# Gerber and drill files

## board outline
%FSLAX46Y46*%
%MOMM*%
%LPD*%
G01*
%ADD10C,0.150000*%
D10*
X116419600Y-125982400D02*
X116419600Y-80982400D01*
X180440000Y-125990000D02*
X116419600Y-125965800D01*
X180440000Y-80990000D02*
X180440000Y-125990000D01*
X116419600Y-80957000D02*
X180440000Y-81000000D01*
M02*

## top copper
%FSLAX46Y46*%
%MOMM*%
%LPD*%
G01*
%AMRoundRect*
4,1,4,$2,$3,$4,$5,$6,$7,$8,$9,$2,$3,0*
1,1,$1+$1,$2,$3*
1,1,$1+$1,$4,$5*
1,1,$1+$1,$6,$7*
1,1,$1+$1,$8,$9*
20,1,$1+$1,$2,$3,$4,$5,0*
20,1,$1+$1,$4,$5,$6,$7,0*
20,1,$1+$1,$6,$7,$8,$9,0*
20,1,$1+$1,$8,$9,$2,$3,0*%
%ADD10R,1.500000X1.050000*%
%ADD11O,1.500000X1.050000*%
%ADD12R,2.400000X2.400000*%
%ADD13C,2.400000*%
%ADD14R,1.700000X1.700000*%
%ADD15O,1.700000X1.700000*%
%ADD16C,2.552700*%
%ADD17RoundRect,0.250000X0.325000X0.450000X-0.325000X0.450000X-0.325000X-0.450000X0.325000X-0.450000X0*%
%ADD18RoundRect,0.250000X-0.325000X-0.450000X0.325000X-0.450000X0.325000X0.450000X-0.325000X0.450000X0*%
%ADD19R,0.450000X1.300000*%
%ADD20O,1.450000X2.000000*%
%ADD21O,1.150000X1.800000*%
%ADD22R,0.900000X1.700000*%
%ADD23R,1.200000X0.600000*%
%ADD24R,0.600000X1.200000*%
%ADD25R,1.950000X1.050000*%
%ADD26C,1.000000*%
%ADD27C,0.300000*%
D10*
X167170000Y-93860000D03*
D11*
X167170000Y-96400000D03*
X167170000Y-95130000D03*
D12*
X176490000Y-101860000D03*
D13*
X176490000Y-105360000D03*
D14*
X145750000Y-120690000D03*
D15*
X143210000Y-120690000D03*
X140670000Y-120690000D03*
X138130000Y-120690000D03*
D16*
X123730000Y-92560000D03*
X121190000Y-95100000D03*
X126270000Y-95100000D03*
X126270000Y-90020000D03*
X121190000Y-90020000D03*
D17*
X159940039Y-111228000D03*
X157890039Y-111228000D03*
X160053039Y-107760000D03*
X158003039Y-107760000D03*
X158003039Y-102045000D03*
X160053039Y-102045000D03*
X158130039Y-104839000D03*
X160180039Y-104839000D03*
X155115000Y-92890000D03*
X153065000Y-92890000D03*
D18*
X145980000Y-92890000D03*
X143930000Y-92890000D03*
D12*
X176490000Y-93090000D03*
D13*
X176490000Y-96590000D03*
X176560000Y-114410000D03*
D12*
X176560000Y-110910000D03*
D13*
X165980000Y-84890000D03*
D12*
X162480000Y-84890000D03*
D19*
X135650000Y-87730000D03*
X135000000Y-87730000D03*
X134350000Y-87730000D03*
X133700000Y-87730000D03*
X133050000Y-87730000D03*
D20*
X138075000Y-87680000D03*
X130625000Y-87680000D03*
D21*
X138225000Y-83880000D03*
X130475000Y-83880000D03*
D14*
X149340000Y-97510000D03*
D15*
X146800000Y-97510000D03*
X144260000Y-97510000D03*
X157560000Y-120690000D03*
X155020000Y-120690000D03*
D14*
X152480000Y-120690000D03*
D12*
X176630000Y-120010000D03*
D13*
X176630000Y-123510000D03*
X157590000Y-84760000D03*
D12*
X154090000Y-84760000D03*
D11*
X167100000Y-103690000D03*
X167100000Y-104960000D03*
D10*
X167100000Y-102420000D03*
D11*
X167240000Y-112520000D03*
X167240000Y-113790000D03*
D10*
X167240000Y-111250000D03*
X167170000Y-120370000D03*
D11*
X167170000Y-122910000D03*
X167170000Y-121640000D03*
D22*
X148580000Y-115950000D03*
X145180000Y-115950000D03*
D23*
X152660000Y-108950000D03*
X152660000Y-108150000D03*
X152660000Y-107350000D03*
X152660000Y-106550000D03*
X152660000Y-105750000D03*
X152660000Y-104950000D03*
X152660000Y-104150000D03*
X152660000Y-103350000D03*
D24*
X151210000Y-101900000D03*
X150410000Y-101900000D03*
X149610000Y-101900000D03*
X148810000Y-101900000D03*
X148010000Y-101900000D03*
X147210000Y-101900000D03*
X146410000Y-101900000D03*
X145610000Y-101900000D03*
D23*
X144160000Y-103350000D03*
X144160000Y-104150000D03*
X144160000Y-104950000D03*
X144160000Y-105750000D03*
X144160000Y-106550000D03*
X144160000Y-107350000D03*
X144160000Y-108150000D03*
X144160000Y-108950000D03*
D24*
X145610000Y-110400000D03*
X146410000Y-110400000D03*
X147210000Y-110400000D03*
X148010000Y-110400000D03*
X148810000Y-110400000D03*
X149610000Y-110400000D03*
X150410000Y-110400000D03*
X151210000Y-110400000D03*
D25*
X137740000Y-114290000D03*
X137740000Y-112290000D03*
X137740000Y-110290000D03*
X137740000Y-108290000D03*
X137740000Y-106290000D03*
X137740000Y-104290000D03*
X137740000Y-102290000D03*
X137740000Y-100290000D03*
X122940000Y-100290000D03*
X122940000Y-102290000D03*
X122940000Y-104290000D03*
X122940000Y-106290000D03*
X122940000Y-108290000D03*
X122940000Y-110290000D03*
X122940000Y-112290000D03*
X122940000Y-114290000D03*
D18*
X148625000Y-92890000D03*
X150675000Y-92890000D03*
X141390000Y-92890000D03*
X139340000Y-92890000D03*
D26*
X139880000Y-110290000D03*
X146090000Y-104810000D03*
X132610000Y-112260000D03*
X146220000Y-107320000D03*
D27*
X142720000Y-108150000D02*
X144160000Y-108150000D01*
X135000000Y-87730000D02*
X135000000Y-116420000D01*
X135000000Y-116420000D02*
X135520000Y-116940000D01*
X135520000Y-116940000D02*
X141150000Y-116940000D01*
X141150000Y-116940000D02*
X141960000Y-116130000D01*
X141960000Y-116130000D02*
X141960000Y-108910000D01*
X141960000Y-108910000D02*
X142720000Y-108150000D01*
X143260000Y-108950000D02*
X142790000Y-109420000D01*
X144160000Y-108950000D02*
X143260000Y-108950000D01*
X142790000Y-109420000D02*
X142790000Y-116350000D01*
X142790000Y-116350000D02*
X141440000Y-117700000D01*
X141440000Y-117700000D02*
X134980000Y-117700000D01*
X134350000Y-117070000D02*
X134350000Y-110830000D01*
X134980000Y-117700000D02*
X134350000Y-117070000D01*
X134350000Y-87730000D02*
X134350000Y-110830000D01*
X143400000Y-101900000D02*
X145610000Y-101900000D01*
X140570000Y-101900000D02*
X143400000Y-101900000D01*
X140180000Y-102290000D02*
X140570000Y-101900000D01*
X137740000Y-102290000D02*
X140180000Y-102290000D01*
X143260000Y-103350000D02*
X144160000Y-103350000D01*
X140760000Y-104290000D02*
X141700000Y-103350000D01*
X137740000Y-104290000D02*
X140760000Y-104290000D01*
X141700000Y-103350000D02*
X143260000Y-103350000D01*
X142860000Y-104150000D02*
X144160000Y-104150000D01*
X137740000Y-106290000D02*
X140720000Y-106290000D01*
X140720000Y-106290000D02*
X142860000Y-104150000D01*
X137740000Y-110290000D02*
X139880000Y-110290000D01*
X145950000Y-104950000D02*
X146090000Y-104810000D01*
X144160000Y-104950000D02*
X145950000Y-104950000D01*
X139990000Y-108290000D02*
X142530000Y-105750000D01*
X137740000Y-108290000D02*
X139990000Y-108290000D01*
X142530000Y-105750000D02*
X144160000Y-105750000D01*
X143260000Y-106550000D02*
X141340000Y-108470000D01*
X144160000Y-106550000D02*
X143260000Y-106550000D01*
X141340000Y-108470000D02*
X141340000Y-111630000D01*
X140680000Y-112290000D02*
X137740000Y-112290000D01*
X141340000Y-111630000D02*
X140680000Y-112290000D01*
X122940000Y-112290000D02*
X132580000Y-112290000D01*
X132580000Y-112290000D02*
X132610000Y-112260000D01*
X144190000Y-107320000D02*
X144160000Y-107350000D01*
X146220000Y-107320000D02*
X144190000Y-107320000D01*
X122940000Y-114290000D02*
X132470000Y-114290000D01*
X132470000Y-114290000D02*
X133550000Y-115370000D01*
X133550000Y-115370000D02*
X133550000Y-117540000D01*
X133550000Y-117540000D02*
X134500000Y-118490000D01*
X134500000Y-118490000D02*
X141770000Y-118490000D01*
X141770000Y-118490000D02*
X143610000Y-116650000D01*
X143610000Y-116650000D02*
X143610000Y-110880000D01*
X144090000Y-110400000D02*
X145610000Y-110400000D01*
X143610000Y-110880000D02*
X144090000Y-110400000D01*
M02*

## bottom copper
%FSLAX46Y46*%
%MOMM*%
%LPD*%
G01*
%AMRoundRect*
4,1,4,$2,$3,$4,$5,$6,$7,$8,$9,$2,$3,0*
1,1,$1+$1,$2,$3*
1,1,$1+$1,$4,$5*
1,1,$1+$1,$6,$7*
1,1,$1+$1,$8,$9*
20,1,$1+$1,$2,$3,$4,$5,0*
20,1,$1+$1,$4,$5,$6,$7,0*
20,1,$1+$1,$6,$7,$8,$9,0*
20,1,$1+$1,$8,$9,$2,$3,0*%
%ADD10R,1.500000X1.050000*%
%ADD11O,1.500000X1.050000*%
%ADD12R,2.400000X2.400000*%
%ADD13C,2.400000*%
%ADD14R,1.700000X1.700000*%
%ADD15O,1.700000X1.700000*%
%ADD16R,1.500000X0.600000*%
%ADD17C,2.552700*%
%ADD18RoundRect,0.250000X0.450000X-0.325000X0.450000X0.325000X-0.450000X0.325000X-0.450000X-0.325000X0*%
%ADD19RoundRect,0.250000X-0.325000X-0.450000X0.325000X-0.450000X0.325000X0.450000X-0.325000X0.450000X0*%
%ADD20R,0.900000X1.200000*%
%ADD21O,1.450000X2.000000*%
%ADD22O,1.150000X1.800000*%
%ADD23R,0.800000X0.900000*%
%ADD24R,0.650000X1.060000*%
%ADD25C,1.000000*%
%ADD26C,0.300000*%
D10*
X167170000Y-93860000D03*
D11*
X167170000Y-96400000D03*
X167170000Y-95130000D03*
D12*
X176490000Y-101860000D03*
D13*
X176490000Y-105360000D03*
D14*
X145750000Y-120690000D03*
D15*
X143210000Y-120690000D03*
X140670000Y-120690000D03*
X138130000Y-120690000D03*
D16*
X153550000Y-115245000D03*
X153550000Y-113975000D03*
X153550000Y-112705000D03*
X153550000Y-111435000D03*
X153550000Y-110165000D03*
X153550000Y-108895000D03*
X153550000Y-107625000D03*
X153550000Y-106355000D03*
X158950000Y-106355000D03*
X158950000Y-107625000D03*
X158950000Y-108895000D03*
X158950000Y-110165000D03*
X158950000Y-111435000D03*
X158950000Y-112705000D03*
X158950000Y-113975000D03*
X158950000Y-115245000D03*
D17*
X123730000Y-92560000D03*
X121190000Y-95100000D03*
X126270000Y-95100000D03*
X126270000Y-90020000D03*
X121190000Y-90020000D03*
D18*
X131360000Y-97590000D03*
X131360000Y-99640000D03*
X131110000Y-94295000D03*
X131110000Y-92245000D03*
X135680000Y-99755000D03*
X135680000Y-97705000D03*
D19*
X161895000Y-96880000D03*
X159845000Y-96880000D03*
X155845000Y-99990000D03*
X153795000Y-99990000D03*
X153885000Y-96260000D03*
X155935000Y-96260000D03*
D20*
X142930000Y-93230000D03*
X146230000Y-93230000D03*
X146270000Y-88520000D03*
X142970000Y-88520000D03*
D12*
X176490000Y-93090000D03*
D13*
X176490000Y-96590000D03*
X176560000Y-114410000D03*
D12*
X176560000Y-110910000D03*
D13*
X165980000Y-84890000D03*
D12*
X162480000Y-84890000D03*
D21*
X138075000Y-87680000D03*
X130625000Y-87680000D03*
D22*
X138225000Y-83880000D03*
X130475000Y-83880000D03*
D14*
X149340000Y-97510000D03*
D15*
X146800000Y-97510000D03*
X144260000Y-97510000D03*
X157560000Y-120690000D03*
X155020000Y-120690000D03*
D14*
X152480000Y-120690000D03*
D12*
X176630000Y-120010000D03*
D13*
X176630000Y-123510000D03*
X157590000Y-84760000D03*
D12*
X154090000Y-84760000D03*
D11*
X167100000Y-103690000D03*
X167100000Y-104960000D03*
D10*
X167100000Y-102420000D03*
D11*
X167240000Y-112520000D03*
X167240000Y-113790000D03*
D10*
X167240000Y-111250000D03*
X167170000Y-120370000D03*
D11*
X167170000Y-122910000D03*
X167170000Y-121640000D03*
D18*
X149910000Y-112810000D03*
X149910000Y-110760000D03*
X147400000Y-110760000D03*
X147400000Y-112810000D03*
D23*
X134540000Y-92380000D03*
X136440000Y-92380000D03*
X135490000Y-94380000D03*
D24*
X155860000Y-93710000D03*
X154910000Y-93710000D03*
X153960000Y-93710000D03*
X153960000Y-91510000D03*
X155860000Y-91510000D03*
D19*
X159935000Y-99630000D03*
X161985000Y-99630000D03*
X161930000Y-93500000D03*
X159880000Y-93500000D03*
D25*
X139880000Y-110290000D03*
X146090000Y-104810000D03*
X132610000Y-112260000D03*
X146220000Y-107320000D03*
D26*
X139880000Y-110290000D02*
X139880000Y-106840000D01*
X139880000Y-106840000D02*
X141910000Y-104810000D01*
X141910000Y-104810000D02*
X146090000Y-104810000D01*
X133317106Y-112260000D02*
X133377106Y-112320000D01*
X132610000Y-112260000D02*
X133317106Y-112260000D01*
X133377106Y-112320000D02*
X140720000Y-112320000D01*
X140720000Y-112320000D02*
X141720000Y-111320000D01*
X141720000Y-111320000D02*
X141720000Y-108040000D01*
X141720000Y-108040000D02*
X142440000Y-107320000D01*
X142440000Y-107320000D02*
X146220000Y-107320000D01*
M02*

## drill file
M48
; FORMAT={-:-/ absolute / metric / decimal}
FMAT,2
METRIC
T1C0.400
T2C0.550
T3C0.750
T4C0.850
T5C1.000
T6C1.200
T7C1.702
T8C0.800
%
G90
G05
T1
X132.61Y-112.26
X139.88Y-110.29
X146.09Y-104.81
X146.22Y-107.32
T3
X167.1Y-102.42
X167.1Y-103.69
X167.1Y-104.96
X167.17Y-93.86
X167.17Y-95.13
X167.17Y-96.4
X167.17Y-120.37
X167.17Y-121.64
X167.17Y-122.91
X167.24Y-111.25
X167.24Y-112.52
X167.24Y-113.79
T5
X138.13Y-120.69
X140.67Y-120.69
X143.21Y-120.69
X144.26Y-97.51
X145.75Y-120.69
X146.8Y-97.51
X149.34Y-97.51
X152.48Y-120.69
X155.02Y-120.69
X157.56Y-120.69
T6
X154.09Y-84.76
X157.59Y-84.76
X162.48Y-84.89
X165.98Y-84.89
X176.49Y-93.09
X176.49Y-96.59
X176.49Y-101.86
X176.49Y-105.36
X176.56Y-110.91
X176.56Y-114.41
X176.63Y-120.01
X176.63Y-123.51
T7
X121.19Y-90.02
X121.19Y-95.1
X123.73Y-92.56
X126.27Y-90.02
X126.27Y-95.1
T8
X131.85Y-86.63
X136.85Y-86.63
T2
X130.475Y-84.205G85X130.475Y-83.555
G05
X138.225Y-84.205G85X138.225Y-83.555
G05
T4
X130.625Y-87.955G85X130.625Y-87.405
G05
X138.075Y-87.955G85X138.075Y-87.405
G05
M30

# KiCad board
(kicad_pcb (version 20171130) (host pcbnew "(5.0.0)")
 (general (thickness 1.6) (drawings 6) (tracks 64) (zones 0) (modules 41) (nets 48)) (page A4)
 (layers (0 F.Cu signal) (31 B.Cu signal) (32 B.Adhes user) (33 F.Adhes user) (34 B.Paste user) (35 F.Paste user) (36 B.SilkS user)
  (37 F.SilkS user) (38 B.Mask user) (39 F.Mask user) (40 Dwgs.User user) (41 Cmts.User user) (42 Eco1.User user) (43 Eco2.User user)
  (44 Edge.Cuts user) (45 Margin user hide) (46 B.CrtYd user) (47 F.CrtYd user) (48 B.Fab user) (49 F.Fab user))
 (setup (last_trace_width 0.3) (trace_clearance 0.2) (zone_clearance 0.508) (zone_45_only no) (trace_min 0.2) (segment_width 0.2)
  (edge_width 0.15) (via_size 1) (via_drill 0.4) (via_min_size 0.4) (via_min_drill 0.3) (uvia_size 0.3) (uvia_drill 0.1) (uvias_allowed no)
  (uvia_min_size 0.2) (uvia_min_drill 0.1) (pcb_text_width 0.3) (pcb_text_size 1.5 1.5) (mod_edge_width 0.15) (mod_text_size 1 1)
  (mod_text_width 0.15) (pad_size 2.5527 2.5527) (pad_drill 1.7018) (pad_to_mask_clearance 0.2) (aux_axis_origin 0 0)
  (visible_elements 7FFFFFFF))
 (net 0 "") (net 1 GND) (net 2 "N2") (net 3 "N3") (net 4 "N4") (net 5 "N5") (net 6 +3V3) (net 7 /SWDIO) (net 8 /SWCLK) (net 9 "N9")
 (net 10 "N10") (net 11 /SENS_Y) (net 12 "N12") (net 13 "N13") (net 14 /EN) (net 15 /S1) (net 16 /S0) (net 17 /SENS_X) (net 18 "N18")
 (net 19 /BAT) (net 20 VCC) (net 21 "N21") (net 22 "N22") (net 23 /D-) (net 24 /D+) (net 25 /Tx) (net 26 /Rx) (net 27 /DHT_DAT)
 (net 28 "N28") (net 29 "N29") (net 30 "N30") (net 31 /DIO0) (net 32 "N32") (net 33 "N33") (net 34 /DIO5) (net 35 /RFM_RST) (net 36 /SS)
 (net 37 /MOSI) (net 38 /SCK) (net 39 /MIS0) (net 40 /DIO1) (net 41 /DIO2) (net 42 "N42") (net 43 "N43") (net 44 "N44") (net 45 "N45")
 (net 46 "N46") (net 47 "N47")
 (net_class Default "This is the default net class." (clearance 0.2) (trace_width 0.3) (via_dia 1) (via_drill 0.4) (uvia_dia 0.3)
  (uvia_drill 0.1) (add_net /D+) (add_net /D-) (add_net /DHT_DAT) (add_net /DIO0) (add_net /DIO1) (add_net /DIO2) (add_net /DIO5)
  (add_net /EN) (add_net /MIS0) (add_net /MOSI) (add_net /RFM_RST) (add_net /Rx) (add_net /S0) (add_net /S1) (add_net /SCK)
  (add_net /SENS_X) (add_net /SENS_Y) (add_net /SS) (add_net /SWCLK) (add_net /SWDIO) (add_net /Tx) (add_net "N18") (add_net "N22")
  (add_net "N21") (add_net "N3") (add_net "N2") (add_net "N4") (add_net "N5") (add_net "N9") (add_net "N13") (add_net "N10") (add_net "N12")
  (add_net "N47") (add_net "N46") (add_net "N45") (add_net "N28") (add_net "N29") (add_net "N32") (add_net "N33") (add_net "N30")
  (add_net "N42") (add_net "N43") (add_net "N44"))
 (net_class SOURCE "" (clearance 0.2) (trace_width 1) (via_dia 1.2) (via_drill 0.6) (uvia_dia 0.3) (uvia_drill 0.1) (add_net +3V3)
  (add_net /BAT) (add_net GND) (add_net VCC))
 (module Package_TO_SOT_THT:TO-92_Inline (layer F.Cu) (at 167.17 93.86 270)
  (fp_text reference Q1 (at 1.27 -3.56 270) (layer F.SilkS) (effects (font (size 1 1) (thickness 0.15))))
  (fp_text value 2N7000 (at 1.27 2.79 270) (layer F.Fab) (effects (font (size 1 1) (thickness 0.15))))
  (pad 1 thru_hole rect (at 0 0 270) (size 1.05 1.5) (drill 0.75) (layers *.Cu *.Mask) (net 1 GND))
  (pad 3 thru_hole oval (at 2.54 0 270) (size 1.05 1.5) (drill 0.75) (layers *.Cu *.Mask) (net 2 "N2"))
  (pad 2 thru_hole oval (at 1.27 0 270) (size 1.05 1.5) (drill 0.75) (layers *.Cu *.Mask) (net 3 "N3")))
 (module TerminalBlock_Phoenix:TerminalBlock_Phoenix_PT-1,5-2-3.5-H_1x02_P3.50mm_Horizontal (layer F.Cu) (at 176.49 101.86 270)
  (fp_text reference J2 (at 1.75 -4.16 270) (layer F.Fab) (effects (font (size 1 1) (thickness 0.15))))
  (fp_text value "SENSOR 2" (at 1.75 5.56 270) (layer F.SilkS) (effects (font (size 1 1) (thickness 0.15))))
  (pad 1 thru_hole rect (at 0 0 270) (size 2.4 2.4) (drill 1.2) (layers *.Cu *.Mask) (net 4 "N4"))
  (pad 2 thru_hole circle (at 3.5 0 270) (size 2.4 2.4) (drill 1.2) (layers *.Cu *.Mask) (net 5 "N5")))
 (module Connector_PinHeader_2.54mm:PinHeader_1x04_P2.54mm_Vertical (layer F.Cu) (at 145.75 120.69 270)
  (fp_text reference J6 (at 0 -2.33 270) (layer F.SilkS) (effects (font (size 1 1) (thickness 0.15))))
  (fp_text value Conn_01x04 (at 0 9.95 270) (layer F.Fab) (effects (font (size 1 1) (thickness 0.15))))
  (pad 1 thru_hole rect (at 0 0 270) (size 1.7 1.7) (drill 1) (layers *.Cu *.Mask) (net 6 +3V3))
  (pad 2 thru_hole oval (at 0 2.54 270) (size 1.7 1.7) (drill 1) (layers *.Cu *.Mask) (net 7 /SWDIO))
  (pad 3 thru_hole oval (at 0 5.08 270) (size 1.7 1.7) (drill 1) (layers *.Cu *.Mask) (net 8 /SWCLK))
  (pad 4 thru_hole oval (at 0 7.62 270) (size 1.7 1.7) (drill 1) (layers *.Cu *.Mask) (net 1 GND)))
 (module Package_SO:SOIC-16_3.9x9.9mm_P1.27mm (layer B.Cu) (at 156.25 110.8)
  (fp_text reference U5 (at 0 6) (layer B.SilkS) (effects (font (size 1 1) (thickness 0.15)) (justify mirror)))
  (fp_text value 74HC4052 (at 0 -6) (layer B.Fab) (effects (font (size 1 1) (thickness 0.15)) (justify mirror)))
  (pad 1 smd rect (at -2.7 4.445) (size 1.5 0.6) (layers B.Cu B.Paste B.Mask) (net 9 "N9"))
  (pad 2 smd rect (at -2.7 3.175) (size 1.5 0.6) (layers B.Cu B.Paste B.Mask) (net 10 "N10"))
  (pad 3 smd rect (at -2.7 1.905) (size 1.5 0.6) (layers B.Cu B.Paste B.Mask) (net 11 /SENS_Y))
  (pad 4 smd rect (at -2.7 0.635) (size 1.5 0.6) (layers B.Cu B.Paste B.Mask) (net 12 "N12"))
  (pad 5 smd rect (at -2.7 -0.635) (size 1.5 0.6) (layers B.Cu B.Paste B.Mask) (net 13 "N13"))
  (pad 6 smd rect (at -2.7 -1.905) (size 1.5 0.6) (layers B.Cu B.Paste B.Mask) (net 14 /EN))
  (pad 7 smd rect (at -2.7 -3.175) (size 1.5 0.6) (layers B.Cu B.Paste B.Mask) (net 1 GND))
  (pad 8 smd rect (at -2.7 -4.445) (size 1.5 0.6) (layers B.Cu B.Paste B.Mask) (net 1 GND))
  (pad 9 smd rect (at 2.7 -4.445) (size 1.5 0.6) (layers B.Cu B.Paste B.Mask) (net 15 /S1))
  (pad 10 smd rect (at 2.7 -3.175) (size 1.5 0.6) (layers B.Cu B.Paste B.Mask) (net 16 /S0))
  (pad 11 smd rect (at 2.7 -1.905) (size 1.5 0.6) (layers B.Cu B.Paste B.Mask) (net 5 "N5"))
  (pad 12 smd rect (at 2.7 -0.635) (size 1.5 0.6) (layers B.Cu B.Paste B.Mask) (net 3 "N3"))
  (pad 13 smd rect (at 2.7 0.635) (size 1.5 0.6) (layers B.Cu B.Paste B.Mask) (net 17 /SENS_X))
  (pad 14 smd rect (at 2.7 1.905) (size 1.5 0.6) (layers B.Cu B.Paste B.Mask) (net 2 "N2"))
  (pad 15 smd rect (at 2.7 3.175) (size 1.5 0.6) (layers B.Cu B.Paste B.Mask) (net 4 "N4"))
  (pad 16 smd rect (at 2.7 4.445) (size 1.5 0.6) (layers B.Cu B.Paste B.Mask) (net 6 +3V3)))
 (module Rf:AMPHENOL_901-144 (layer F.Cu) (at 123.73 92.56 90) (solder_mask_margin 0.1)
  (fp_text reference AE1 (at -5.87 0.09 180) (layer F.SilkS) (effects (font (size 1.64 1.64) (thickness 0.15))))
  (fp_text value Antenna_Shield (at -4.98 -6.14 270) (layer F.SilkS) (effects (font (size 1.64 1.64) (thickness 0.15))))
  (pad 1 thru_hole circle (at 0 0 90) (size 2.5527 2.5527) (drill 1.7018) (layers *.Cu *.Mask F.SilkS) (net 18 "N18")
   (solder_mask_margin 0.2))
  (pad 2 thru_hole circle (at -2.54 -2.54 90) (size 2.5527 2.5527) (drill 1.7018) (layers *.Cu *.Mask F.SilkS) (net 1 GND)
   (solder_mask_margin 0.2))
  (pad E thru_hole circle (at -2.54 2.54 90) (size 2.5527 2.5527) (drill 1.7018) (layers *.Cu *.Mask F.SilkS) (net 1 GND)
   (solder_mask_margin 0.2))
  (pad 4 thru_hole circle (at 2.54 2.54 90) (size 2.5527 2.5527) (drill 1.7018) (layers *.Cu *.Mask F.SilkS) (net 1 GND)
   (solder_mask_margin 0.2))
  (pad 5 thru_hole circle (at 2.54 -2.54 90) (size 2.5527 2.5527) (drill 1.7018) (layers *.Cu *.Mask F.SilkS) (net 1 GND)
   (solder_mask_margin 0.2)))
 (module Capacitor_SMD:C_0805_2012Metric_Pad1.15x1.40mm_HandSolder (layer F.Cu) (at 158.915039 111.228 180)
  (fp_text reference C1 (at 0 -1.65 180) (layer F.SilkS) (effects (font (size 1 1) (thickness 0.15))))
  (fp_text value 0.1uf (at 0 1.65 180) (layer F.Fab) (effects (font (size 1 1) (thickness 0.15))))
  (pad 1 smd roundrect (at -1.025 0 180) (size 1.15 1.4) (layers F.Cu F.Paste F.Mask) (roundrect_rratio 0.217391) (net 6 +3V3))
  (pad 2 smd roundrect (at 1.025 0 180) (size 1.15 1.4) (layers F.Cu F.Paste F.Mask) (roundrect_rratio 0.217391) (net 1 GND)))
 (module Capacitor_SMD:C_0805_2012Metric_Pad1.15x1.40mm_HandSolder (layer B.Cu) (at 131.36 98.615 90)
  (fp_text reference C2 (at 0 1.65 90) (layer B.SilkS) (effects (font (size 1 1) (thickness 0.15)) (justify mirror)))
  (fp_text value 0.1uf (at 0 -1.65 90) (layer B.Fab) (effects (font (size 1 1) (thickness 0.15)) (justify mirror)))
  (pad 2 smd roundrect (at 1.025 0 90) (size 1.15 1.4) (layers B.Cu B.Paste B.Mask) (roundrect_rratio 0.217391) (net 1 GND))
  (pad 1 smd roundrect (at -1.025 0 90) (size 1.15 1.4) (layers B.Cu B.Paste B.Mask) (roundrect_rratio 0.217391) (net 6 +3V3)))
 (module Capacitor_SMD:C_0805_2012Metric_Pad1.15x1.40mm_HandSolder (layer F.Cu) (at 159.028039 107.76 180)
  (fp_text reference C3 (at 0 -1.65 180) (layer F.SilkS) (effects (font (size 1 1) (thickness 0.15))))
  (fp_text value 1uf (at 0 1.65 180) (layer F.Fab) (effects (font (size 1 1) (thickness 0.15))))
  (pad 1 smd roundrect (at -1.025 0 180) (size 1.15 1.4) (layers F.Cu F.Paste F.Mask) (roundrect_rratio 0.217391) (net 6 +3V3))
  (pad 2 smd roundrect (at 1.025 0 180) (size 1.15 1.4) (layers F.Cu F.Paste F.Mask) (roundrect_rratio 0.217391) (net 1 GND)))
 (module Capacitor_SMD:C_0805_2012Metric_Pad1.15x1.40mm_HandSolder (layer B.Cu) (at 131.11 93.27 90)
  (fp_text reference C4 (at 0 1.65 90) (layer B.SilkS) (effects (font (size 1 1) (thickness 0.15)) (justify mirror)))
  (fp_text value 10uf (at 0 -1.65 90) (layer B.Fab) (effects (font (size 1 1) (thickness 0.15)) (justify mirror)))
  (pad 1 smd roundrect (at -1.025 0 90) (size 1.15 1.4) (layers B.Cu B.Paste B.Mask) (roundrect_rratio 0.217391) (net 6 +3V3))
  (pad 2 smd roundrect (at 1.025 0 90) (size 1.15 1.4) (layers B.Cu B.Paste B.Mask) (roundrect_rratio 0.217391) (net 1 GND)))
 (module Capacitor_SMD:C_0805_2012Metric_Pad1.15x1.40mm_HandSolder (layer B.Cu) (at 135.68 98.73 90)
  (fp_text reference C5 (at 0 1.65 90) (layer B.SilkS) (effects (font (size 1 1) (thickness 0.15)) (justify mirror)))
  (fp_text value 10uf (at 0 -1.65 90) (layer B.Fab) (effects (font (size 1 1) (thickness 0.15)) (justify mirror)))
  (pad 1 smd roundrect (at -1.025 0 90) (size 1.15 1.4) (layers B.Cu B.Paste B.Mask) (roundrect_rratio 0.217391) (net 6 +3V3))
  (pad 2 smd roundrect (at 1.025 0 90) (size 1.15 1.4) (layers B.Cu B.Paste B.Mask) (roundrect_rratio 0.217391) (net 1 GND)))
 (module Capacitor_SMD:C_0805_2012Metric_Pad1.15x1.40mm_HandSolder (layer B.Cu) (at 160.87 96.88)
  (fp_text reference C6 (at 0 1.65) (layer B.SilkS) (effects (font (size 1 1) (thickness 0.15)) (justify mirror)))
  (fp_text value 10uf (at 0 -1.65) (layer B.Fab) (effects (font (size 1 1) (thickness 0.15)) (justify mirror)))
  (pad 2 smd roundrect (at 1.025 0) (size 1.15 1.4) (layers B.Cu B.Paste B.Mask) (roundrect_rratio 0.217391) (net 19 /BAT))
  (pad 1 smd roundrect (at -1.025 0) (size 1.15 1.4) (layers B.Cu B.Paste B.Mask) (roundrect_rratio 0.217391) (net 1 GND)))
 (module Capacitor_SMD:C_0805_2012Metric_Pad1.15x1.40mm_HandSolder (layer F.Cu) (at 159.028039 102.045 180)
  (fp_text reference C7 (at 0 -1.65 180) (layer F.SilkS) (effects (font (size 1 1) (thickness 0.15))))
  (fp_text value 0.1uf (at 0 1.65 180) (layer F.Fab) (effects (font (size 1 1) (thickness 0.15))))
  (pad 2 smd roundrect (at 1.025 0 180) (size 1.15 1.4) (layers F.Cu F.Paste F.Mask) (roundrect_rratio 0.217391) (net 1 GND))
  (pad 1 smd roundrect (at -1.025 0 180) (size 1.15 1.4) (layers F.Cu F.Paste F.Mask) (roundrect_rratio 0.217391) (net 6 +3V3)))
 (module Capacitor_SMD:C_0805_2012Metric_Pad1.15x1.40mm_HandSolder (layer F.Cu) (at 159.155039 104.839 180)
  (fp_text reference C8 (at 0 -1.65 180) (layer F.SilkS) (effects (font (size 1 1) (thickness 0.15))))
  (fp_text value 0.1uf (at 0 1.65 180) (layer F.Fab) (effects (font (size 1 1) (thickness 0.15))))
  (pad 2 smd roundrect (at 1.025 0 180) (size 1.15 1.4) (layers F.Cu F.Paste F.Mask) (roundrect_rratio 0.217391) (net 1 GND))
  (pad 1 smd roundrect (at -1.025 0 180) (size 1.15 1.4) (layers F.Cu F.Paste F.Mask) (roundrect_rratio 0.217391) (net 6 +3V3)))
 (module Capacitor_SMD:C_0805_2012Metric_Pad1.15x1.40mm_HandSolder (layer B.Cu) (at 154.82 99.99)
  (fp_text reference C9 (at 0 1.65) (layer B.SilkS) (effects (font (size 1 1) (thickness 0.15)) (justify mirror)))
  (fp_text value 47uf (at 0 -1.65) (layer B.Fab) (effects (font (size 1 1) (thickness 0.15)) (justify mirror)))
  (pad 2 smd roundrect (at 1.025 0) (size 1.15 1.4) (layers B.Cu B.Paste B.Mask) (roundrect_rratio 0.217391) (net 1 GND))
  (pad 1 smd roundrect (at -1.025 0) (size 1.15 1.4) (layers B.Cu B.Paste B.Mask) (roundrect_rratio 0.217391) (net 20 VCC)))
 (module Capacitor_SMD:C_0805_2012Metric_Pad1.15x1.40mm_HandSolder (layer B.Cu) (at 154.91 96.26)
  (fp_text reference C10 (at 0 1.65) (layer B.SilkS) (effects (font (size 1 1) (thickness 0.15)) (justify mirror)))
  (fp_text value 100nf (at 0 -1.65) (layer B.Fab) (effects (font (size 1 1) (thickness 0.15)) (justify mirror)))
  (pad 1 smd roundrect (at -1.025 0) (size 1.15 1.4) (layers B.Cu B.Paste B.Mask) (roundrect_rratio 0.217391) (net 20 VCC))
  (pad 2 smd roundrect (at 1.025 0) (size 1.15 1.4) (layers B.Cu B.Paste B.Mask) (roundrect_rratio 0.217391) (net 1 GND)))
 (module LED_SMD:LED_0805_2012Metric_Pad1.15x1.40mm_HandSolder (layer F.Cu) (at 154.09 92.89 180)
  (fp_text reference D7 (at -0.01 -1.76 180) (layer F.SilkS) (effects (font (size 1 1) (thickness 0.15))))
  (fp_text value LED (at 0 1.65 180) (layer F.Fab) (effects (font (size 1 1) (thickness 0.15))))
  (pad 1 smd roundrect (at -1.025 0 180) (size 1.15 1.4) (layers F.Cu F.Paste F.Mask) (roundrect_rratio 0.217391) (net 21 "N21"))
  (pad 2 smd roundrect (at 1.025 0 180) (size 1.15 1.4) (layers F.Cu F.Paste F.Mask) (roundrect_rratio 0.217391) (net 20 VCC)))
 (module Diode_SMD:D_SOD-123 (layer B.Cu) (at 144.58 93.23)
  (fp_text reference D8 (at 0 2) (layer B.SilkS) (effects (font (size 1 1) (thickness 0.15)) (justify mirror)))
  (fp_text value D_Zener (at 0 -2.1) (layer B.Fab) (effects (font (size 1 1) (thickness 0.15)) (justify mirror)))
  (pad 1 smd rect (at -1.65 0) (size 0.9 1.2) (layers B.Cu B.Paste B.Mask) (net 6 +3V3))
  (pad 2 smd rect (at 1.65 0) (size 0.9 1.2) (layers B.Cu B.Paste B.Mask) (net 20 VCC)))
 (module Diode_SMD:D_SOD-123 (layer B.Cu) (at 144.62 88.52)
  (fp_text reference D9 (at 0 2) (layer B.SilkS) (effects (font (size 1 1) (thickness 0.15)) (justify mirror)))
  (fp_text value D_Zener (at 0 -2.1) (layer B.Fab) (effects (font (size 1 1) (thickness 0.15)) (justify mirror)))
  (pad 2 smd rect (at 1.65 0) (size 0.9 1.2) (layers B.Cu B.Paste B.Mask) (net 19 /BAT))
  (pad 1 smd rect (at -1.65 0) (size 0.9 1.2) (layers B.Cu B.Paste B.Mask) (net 6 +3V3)))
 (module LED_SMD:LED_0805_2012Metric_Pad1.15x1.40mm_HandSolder (layer F.Cu) (at 144.955 92.89)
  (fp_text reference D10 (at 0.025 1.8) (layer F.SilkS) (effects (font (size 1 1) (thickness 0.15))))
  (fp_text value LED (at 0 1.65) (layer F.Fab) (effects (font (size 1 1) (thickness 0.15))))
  (pad 2 smd roundrect (at 1.025 0) (size 1.15 1.4) (layers F.Cu F.Paste F.Mask) (roundrect_rratio 0.217391) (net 6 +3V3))
  (pad 1 smd roundrect (at -1.025 0) (size 1.15 1.4) (layers F.Cu F.Paste F.Mask) (roundrect_rratio 0.217391) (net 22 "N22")))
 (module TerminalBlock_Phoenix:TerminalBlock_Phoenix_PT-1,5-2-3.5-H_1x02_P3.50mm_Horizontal (layer F.Cu) (at 176.49 93.09 270)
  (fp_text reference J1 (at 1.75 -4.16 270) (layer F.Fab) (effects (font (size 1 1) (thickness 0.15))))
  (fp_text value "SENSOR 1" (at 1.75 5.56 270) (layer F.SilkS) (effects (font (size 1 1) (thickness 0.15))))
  (pad 1 thru_hole rect (at 0 0 270) (size 2.4 2.4) (drill 1.2) (layers *.Cu *.Mask) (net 3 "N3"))
  (pad 2 thru_hole circle (at 3.5 0 270) (size 2.4 2.4) (drill 1.2) (layers *.Cu *.Mask) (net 2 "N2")))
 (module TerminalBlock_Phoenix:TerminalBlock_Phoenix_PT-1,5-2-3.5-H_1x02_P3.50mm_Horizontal (layer F.Cu) (at 176.56 110.91 270)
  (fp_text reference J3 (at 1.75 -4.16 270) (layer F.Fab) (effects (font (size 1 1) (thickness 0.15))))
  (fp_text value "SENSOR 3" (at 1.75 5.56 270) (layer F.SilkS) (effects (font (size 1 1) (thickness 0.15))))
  (pad 2 thru_hole circle (at 3.5 0 270) (size 2.4 2.4) (drill 1.2) (layers *.Cu *.Mask) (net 13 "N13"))
  (pad 1 thru_hole rect (at 0 0 270) (size 2.4 2.4) (drill 1.2) (layers *.Cu *.Mask) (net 9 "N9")))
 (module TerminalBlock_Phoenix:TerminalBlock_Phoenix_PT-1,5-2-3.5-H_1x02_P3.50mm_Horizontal (layer F.Cu) (at 162.48 84.89)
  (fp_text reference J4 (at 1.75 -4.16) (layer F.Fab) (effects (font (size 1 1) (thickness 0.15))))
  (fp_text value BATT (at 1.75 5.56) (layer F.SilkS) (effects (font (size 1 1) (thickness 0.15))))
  (pad 2 thru_hole circle (at 3.5 0) (size 2.4 2.4) (drill 1.2) (layers *.Cu *.Mask) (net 1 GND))
  (pad 1 thru_hole rect (at 0 0) (size 2.4 2.4) (drill 1.2) (layers *.Cu *.Mask) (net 19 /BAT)))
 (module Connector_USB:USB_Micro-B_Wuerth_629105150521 (layer F.Cu) (at 134.35 85.83 180)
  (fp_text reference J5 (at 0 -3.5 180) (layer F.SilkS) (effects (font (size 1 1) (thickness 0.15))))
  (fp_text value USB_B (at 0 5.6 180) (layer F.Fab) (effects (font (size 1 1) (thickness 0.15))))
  (pad 1 smd rect (at -1.3 -1.9 180) (size 0.45 1.3) (layers F.Cu F.Paste F.Mask) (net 20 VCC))
  (pad 2 smd rect (at -0.65 -1.9 180) (size 0.45 1.3) (layers F.Cu F.Paste F.Mask) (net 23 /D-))
  (pad 3 smd rect (at 0 -1.9 180) (size 0.45 1.3) (layers F.Cu F.Paste F.Mask) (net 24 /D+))
  (pad 4 smd rect (at 0.65 -1.9 180) (size 0.45 1.3) (layers F.Cu F.Paste F.Mask) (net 1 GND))
  (pad 5 smd rect (at 1.3 -1.9 180) (size 0.45 1.3) (layers F.Cu F.Paste F.Mask) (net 1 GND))
  (pad 6 thru_hole oval (at -3.725 -1.85 180) (size 1.45 2) (drill oval 0.85 1.4) (layers *.Cu *.Mask))
  (pad 6 thru_hole oval (at 3.725 -1.85 180) (size 1.45 2) (drill oval 0.85 1.4) (layers *.Cu *.Mask))
  (pad 6 thru_hole oval (at -3.875 1.95 180) (size 1.15 1.8) (drill oval 0.55 1.2) (layers *.Cu *.Mask))
  (pad 6 thru_hole oval (at 3.875 1.95 180) (size 1.15 1.8) (drill oval 0.55 1.2) (layers *.Cu *.Mask))
  (pad "" np_thru_hole oval (at -2.5 -0.8 180) (size 0.8 0.8) (drill 0.8) (layers *.Cu *.Mask))
  (pad "" np_thru_hole oval (at 2.5 -0.8 180) (size 0.8 0.8) (drill 0.8) (layers *.Cu *.Mask)))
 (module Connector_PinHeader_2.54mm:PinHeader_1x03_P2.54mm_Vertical (layer F.Cu) (at 149.34 97.51 270)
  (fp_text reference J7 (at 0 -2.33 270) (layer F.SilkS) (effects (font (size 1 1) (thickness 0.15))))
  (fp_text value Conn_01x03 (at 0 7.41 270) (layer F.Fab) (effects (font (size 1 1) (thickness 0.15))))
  (pad 1 thru_hole rect (at 0 0 270) (size 1.7 1.7) (drill 1) (layers *.Cu *.Mask) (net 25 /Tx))
  (pad 2 thru_hole oval (at 0 2.54 270) (size 1.7 1.7) (drill 1) (layers *.Cu *.Mask) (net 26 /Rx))
  (pad 3 thru_hole oval (at 0 5.08 270) (size 1.7 1.7) (drill 1) (layers *.Cu *.Mask) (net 1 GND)))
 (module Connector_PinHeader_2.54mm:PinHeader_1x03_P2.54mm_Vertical (layer F.Cu) (at 152.48 120.69 90)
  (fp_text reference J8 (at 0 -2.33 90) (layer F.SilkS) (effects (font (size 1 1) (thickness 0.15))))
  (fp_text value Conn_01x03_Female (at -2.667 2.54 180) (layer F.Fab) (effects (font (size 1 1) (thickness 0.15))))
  (pad 3 thru_hole oval (at 0 5.08 90) (size 1.7 1.7) (drill 1) (layers *.Cu *.Mask) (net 1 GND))
  (pad 2 thru_hole oval (at 0 2.54 90) (size 1.7 1.7) (drill 1) (layers *.Cu *.Mask) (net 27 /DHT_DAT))
  (pad 1 thru_hole rect (at 0 0 90) (size 1.7 1.7) (drill 1) (layers *.Cu *.Mask) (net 6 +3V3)))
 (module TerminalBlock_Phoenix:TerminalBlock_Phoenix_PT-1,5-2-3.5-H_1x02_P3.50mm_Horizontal (layer F.Cu) (at 176.63 120.01 270)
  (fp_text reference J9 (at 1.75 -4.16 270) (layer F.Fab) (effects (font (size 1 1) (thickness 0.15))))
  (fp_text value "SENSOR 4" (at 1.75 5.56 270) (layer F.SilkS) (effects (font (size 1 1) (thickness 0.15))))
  (pad 1 thru_hole rect (at 0 0 270) (size 2.4 2.4) (drill 1.2) (layers *.Cu *.Mask) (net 10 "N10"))
  (pad 2 thru_hole circle (at 3.5 0 270) (size 2.4 2.4) (drill 1.2) (layers *.Cu *.Mask) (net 12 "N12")))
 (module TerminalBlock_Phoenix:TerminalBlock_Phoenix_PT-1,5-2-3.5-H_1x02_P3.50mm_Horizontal (layer F.Cu) (at 154.09 84.76)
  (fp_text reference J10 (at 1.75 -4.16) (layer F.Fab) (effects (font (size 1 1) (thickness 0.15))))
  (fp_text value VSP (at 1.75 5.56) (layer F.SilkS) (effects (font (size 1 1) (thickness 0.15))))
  (pad 2 thru_hole circle (at 3.5 0) (size 2.4 2.4) (drill 1.2) (layers *.Cu *.Mask) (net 20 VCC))
  (pad 1 thru_hole rect (at 0 0) (size 2.4 2.4) (drill 1.2) (layers *.Cu *.Mask) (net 1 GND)))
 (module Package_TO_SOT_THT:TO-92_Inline (layer F.Cu) (at 167.1 102.42 270)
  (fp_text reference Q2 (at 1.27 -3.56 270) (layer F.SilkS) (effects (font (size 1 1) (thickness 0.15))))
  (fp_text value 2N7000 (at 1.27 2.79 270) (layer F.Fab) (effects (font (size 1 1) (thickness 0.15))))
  (pad 2 thru_hole oval (at 1.27 0 270) (size 1.05 1.5) (drill 0.75) (layers *.Cu *.Mask) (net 4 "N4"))
  (pad 3 thru_hole oval (at 2.54 0 270) (size 1.05 1.5) (drill 0.75) (layers *.Cu *.Mask) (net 5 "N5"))
  (pad 1 thru_hole rect (at 0 0 270) (size 1.05 1.5) (drill 0.75) (layers *.Cu *.Mask) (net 1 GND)))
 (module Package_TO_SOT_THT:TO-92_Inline (layer F.Cu) (at 167.24 111.25 270)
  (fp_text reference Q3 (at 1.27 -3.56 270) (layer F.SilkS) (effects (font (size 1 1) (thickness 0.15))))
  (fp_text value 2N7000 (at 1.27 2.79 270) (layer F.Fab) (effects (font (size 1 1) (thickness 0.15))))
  (pad 2 thru_hole oval (at 1.27 0 270) (size 1.05 1.5) (drill 0.75) (layers *.Cu *.Mask) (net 9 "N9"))
  (pad 3 thru_hole oval (at 2.54 0 270) (size 1.05 1.5) (drill 0.75) (layers *.Cu *.Mask) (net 13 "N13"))
  (pad 1 thru_hole rect (at 0 0 270) (size 1.05 1.5) (drill 0.75) (layers *.Cu *.Mask) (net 1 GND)))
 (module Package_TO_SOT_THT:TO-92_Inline (layer F.Cu) (at 167.17 120.37 270)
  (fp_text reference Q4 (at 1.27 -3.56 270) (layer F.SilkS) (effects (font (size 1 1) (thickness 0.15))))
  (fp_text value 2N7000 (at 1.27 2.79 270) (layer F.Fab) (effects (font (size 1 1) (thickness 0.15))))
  (pad 1 thru_hole rect (at 0 0 270) (size 1.05 1.5) (drill 0.75) (layers *.Cu *.Mask) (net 1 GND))
  (pad 3 thru_hole oval (at 2.54 0 270) (size 1.05 1.5) (drill 0.75) (layers *.Cu *.Mask) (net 12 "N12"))
  (pad 2 thru_hole oval (at 1.27 0 270) (size 1.05 1.5) (drill 0.75) (layers *.Cu *.Mask) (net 10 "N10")))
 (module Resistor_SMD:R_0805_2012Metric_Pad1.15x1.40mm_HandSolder (layer B.Cu) (at 149.91 111.785 90)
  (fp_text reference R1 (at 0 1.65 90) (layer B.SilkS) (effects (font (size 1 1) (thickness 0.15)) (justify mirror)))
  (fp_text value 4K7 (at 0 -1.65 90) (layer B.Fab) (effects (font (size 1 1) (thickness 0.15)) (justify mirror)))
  (pad 1 smd roundrect (at -1.025 0 90) (size 1.15 1.4) (layers B.Cu B.Paste B.Mask) (roundrect_rratio 0.217391) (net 17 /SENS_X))
  (pad 2 smd roundrect (at 1.025 0 90) (size 1.15 1.4) (layers B.Cu B.Paste B.Mask) (roundrect_rratio 0.217391) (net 1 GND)))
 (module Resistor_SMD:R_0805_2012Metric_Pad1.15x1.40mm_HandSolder (layer B.Cu) (at 147.4 111.785 90)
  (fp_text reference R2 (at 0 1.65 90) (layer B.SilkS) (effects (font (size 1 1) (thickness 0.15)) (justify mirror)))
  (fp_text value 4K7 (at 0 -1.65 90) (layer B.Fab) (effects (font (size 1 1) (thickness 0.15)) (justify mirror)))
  (pad 2 smd roundrect (at 1.025 0 90) (size 1.15 1.4) (layers B.Cu B.Paste B.Mask) (roundrect_rratio 0.217391) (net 1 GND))
  (pad 1 smd roundrect (at -1.025 0 90) (size 1.15 1.4) (layers B.Cu B.Paste B.Mask) (roundrect_rratio 0.217391) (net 11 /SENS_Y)))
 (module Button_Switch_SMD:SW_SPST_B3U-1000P (layer F.Cu) (at 146.88 115.95 180)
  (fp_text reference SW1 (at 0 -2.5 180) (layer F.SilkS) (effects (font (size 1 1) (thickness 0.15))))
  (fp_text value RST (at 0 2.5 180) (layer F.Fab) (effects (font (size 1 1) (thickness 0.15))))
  (pad 1 smd rect (at -1.7 0 180) (size 0.9 1.7) (layers F.Cu F.Paste F.Mask) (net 1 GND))
  (pad 2 smd rect (at 1.7 0 180) (size 0.9 1.7) (layers F.Cu F.Paste F.Mask) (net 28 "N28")))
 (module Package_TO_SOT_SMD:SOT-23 (layer B.Cu) (at 135.49 93.38 270)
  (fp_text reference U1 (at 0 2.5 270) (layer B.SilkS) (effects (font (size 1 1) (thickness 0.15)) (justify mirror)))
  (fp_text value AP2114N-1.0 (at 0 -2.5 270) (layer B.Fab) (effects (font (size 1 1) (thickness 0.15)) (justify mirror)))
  (pad 1 smd rect (at -1 0.95 270) (size 0.9 0.8) (layers B.Cu B.Paste B.Mask) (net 1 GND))
  (pad 2 smd rect (at -1 -0.95 270) (size 0.9 0.8) (layers B.Cu B.Paste B.Mask) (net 6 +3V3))
  (pad 3 smd rect (at 1 0 270) (size 0.9 0.8) (layers B.Cu B.Paste B.Mask) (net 6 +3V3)))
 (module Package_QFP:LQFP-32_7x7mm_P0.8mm (layer F.Cu) (at 148.41 106.15 180)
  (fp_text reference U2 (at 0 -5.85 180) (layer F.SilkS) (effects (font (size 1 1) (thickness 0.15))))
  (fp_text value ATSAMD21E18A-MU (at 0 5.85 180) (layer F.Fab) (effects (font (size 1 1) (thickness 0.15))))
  (pad 1 smd rect (at -4.25 -2.8 180) (size 1.2 0.6) (layers F.Cu F.Paste F.Mask) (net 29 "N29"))
  (pad 2 smd rect (at -4.25 -2 180) (size 1.2 0.6) (layers F.Cu F.Paste F.Mask) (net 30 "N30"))
  (pad 3 smd rect (at -4.25 -1.2 180) (size 1.2 0.6) (layers F.Cu F.Paste F.Mask) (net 17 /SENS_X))
  (pad 4 smd rect (at -4.25 -0.4 180) (size 1.2 0.6) (layers F.Cu F.Paste F.Mask) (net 27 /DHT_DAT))
  (pad 5 smd rect (at -4.25 0.4 180) (size 1.2 0.6) (layers F.Cu F.Paste F.Mask) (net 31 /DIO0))
  (pad 6 smd rect (at -4.25 1.2 180) (size 1.2 0.6) (layers F.Cu F.Paste F.Mask) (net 11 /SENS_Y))
  (pad 7 smd rect (at -4.25 2 180) (size 1.2 0.6) (layers F.Cu F.Paste F.Mask) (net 16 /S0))
  (pad 8 smd rect (at -4.25 2.8 180) (size 1.2 0.6) (layers F.Cu F.Paste F.Mask) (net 15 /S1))
  (pad 9 smd rect (at -2.8 4.25 270) (size 1.2 0.6) (layers F.Cu F.Paste F.Mask) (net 6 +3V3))
  (pad 10 smd rect (at -2 4.25 270) (size 1.2 0.6) (layers F.Cu F.Paste F.Mask) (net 1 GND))
  (pad 11 smd rect (at -1.2 4.25 270) (size 1.2 0.6) (layers F.Cu F.Paste F.Mask) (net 14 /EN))
  (pad 12 smd rect (at -0.4 4.25 270) (size 1.2 0.6) (layers F.Cu F.Paste F.Mask) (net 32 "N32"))
  (pad 13 smd rect (at 0.4 4.25 270) (size 1.2 0.6) (layers F.Cu F.Paste F.Mask) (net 25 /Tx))
  (pad 14 smd rect (at 1.2 4.25 270) (size 1.2 0.6) (layers F.Cu F.Paste F.Mask) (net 26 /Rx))
  (pad 15 smd rect (at 2 4.25 270) (size 1.2 0.6) (layers F.Cu F.Paste F.Mask) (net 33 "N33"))
  (pad 16 smd rect (at 2.8 4.25 270) (size 1.2 0.6) (layers F.Cu F.Paste F.Mask) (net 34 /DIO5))
  (pad 17 smd rect (at 4.25 2.8 180) (size 1.2 0.6) (layers F.Cu F.Paste F.Mask) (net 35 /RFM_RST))
  (pad 18 smd rect (at 4.25 2 180) (size 1.2 0.6) (layers F.Cu F.Paste F.Mask) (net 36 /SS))
  (pad 19 smd rect (at 4.25 1.2 180) (size 1.2 0.6) (layers F.Cu F.Paste F.Mask) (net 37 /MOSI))
  (pad 20 smd rect (at 4.25 0.4 180) (size 1.2 0.6) (layers F.Cu F.Paste F.Mask) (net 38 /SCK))
  (pad 21 smd rect (at 4.25 -0.4 180) (size 1.2 0.6) (layers F.Cu F.Paste F.Mask) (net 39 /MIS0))
  (pad 22 smd rect (at 4.25 -1.2 180) (size 1.2 0.6) (layers F.Cu F.Paste F.Mask) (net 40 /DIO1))
  (pad 23 smd rect (at 4.25 -2 180) (size 1.2 0.6) (layers F.Cu F.Paste F.Mask) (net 23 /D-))
  (pad 24 smd rect (at 4.25 -2.8 180) (size 1.2 0.6) (layers F.Cu F.Paste F.Mask) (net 24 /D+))
  (pad 25 smd rect (at 2.8 -4.25 270) (size 1.2 0.6) (layers F.Cu F.Paste F.Mask) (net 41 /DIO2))
  (pad 26 smd rect (at 2 -4.25 270) (size 1.2 0.6) (layers F.Cu F.Paste F.Mask) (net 28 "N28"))
  (pad 27 smd rect (at 1.2 -4.25 270) (size 1.2 0.6) (layers F.Cu F.Paste F.Mask) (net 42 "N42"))
  (pad 28 smd rect (at 0.4 -4.25 270) (size 1.2 0.6) (layers F.Cu F.Paste F.Mask) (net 1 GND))
  (pad 29 smd rect (at -0.4 -4.25 270) (size 1.2 0.6) (layers F.Cu F.Paste F.Mask) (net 1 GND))
  (pad 30 smd rect (at -1.2 -4.25 270) (size 1.2 0.6) (layers F.Cu F.Paste F.Mask) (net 6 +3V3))
  (pad 31 smd rect (at -2 -4.25 270) (size 1.2 0.6) (layers F.Cu F.Paste F.Mask) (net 8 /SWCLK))
  (pad 32 smd rect (at -2.8 -4.25 270) (size 1.2 0.6) (layers F.Cu F.Paste F.Mask) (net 7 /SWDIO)))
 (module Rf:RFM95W (layer F.Cu) (at 130.34 107.29 180)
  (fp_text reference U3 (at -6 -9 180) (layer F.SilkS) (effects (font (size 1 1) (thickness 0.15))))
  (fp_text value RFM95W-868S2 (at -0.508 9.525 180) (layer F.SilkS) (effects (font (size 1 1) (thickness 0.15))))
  (pad 1 smd rect (at -7.4 -7 180) (size 1.95 1.05) (layers F.Cu F.Paste F.Mask) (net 1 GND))
  (pad 2 smd rect (at -7.4 -5 180) (size 1.95 1.05) (layers F.Cu F.Paste F.Mask) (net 39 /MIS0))
  (pad 3 smd rect (at -7.4 -3 180) (size 1.95 1.05) (layers F.Cu F.Paste F.Mask) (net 37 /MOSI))
  (pad 4 smd rect (at -7.4 -1 180) (size 1.95 1.05) (layers F.Cu F.Paste F.Mask) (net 38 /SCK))
  (pad 5 smd rect (at -7.4 1 180) (size 1.95 1.05) (layers F.Cu F.Paste F.Mask) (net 36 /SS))
  (pad 6 smd rect (at -7.4 3 180) (size 1.95 1.05) (layers F.Cu F.Paste F.Mask) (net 35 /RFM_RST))
  (pad 7 smd rect (at -7.4 5 180) (size 1.95 1.05) (layers F.Cu F.Paste F.Mask) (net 34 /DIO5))
  (pad 8 smd rect (at -7.4 7 180) (size 1.95 1.05) (layers F.Cu F.Paste F.Mask) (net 1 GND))
  (pad 9 smd rect (at 7.4 7) (size 1.95 1.05) (layers F.Cu F.Paste F.Mask) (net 18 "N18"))
  (pad 10 smd rect (at 7.4 5) (size 1.95 1.05) (layers F.Cu F.Paste F.Mask) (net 1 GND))
  (pad 11 smd rect (at 7.4 3) (size 1.95 1.05) (layers F.Cu F.Paste F.Mask) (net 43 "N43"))
  (pad 12 smd rect (at 7.4 1) (size 1.95 1.05) (layers F.Cu F.Paste F.Mask) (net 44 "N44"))
  (pad 13 smd rect (at 7.4 -1) (size 1.95 1.05) (layers F.Cu F.Paste F.Mask) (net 6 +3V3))
  (pad 14 smd rect (at 7.4 -3) (size 1.95 1.05) (layers F.Cu F.Paste F.Mask) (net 31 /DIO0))
  (pad 15 smd rect (at 7.4 -5) (size 1.95 1.05) (layers F.Cu F.Paste F.Mask) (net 40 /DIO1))
  (pad 16 smd rect (at 7.4 -7) (size 1.95 1.05) (layers F.Cu F.Paste F.Mask) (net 41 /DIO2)))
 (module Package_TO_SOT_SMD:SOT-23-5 (layer B.Cu) (at 154.91 92.61 90)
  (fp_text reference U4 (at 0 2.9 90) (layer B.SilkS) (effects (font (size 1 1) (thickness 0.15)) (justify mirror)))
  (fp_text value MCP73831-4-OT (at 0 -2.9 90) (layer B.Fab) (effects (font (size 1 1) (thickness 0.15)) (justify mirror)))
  (pad 1 smd rect (at -1.1 0.95 90) (size 1.06 0.65) (layers B.Cu B.Paste B.Mask) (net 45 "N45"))
  (pad 2 smd rect (at -1.1 0 90) (size 1.06 0.65) (layers B.Cu B.Paste B.Mask) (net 1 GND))
  (pad 3 smd rect (at -1.1 -0.95 90) (size 1.06 0.65) (layers B.Cu B.Paste B.Mask) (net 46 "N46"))
  (pad 4 smd rect (at 1.1 -0.95 90) (size 1.06 0.65) (layers B.Cu B.Paste B.Mask) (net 20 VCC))
  (pad 5 smd rect (at 1.1 0.95 90) (size 1.06 0.65) (layers B.Cu B.Paste B.Mask) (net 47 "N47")))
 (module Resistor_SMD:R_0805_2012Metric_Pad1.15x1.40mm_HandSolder (layer B.Cu) (at 160.96 99.63)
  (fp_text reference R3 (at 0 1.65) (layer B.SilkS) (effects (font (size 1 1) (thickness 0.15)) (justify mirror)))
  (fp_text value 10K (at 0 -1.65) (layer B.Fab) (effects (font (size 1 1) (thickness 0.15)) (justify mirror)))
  (pad 1 smd roundrect (at -1.025 0) (size 1.15 1.4) (layers B.Cu B.Paste B.Mask) (roundrect_rratio 0.217391) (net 1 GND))
  (pad 2 smd roundrect (at 1.025 0) (size 1.15 1.4) (layers B.Cu B.Paste B.Mask) (roundrect_rratio 0.217391) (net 47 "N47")))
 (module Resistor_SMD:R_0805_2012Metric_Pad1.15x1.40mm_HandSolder (layer B.Cu) (at 160.905 93.5)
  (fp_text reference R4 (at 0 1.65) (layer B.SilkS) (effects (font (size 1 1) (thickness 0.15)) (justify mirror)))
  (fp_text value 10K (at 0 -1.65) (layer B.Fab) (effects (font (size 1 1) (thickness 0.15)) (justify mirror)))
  (pad 2 smd roundrect (at 1.025 0) (size 1.15 1.4) (layers B.Cu B.Paste B.Mask) (roundrect_rratio 0.217391) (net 19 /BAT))
  (pad 1 smd roundrect (at -1.025 0) (size 1.15 1.4) (layers B.Cu B.Paste B.Mask) (roundrect_rratio 0.217391) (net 46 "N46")))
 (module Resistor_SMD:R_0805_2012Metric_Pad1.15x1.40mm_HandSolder (layer F.Cu) (at 149.65 92.89)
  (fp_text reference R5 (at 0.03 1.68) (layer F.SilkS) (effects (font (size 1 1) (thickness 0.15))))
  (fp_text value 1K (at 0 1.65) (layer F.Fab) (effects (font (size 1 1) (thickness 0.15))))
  (pad 1 smd roundrect (at -1.025 0) (size 1.15 1.4) (layers F.Cu F.Paste F.Mask) (roundrect_rratio 0.217391) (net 45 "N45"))
  (pad 2 smd roundrect (at 1.025 0) (size 1.15 1.4) (layers F.Cu F.Paste F.Mask) (roundrect_rratio 0.217391) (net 21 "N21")))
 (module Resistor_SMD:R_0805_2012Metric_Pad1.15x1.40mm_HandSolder (layer F.Cu) (at 140.365 92.89)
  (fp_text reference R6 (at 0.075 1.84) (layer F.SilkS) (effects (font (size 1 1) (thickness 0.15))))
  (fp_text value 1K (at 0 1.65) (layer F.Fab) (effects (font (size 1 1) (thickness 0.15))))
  (pad 2 smd roundrect (at 1.025 0) (size 1.15 1.4) (layers F.Cu F.Paste F.Mask) (roundrect_rratio 0.217391) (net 1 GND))
  (pad 1 smd roundrect (at -1.025 0) (size 1.15 1.4) (layers F.Cu F.Paste F.Mask) (roundrect_rratio 0.217391) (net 22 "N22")))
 (gr_line (start 116.4196 125.9824) (end 116.4196 80.9824) (layer Edge.Cuts) (width 0.15))
 (gr_line (start 180.44 125.99) (end 116.4196 125.9658) (layer Edge.Cuts) (width 0.15))
 (gr_line (start 180.44 80.99) (end 180.44 125.99) (layer Edge.Cuts) (width 0.15))
 (gr_line (start 116.4196 80.957) (end 180.44 81) (layer Edge.Cuts) (width 0.15))
 (segment (start 142.72 108.15) (end 144.16 108.15) (width 0.3) (layer F.Cu) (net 23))
 (segment (start 135 87.73) (end 135 116.42) (width 0.3) (layer F.Cu) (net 23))
 (segment (start 135 116.42) (end 135.52 116.94) (width 0.3) (layer F.Cu) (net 23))
 (segment (start 135.52 116.94) (end 141.15 116.94) (width 0.3) (layer F.Cu) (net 23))
 (segment (start 141.15 116.94) (end 141.96 116.13) (width 0.3) (layer F.Cu) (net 23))
 (segment (start 141.96 116.13) (end 141.96 108.91) (width 0.3) (layer F.Cu) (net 23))
 (segment (start 141.96 108.91) (end 142.72 108.15) (width 0.3) (layer F.Cu) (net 23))
 (segment (start 143.26 108.95) (end 142.79 109.42) (width 0.3) (layer F.Cu) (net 24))
 (segment (start 144.16 108.95) (end 143.26 108.95) (width 0.3) (layer F.Cu) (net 24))
 (segment (start 142.79 109.42) (end 142.79 116.35) (width 0.3) (layer F.Cu) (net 24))
 (segment (start 142.79 116.35) (end 141.44 117.7) (width 0.3) (layer F.Cu) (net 24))
 (segment (start 141.44 117.7) (end 134.98 117.7) (width 0.3) (layer F.Cu) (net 24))
 (segment (start 134.35 117.07) (end 134.35 110.83) (width 0.3) (layer F.Cu) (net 24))
 (segment (start 134.98 117.7) (end 134.35 117.07) (width 0.3) (layer F.Cu) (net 24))
 (segment (start 134.35 87.73) (end 134.35 110.83) (width 0.3) (layer F.Cu) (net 24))
 (segment (start 143.4 101.9) (end 145.61 101.9) (width 0.3) (layer F.Cu) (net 34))
 (segment (start 140.57 101.9) (end 143.4 101.9) (width 0.3) (layer F.Cu) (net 34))
 (segment (start 140.18 102.29) (end 140.57 101.9) (width 0.3) (layer F.Cu) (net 34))
 (segment (start 137.74 102.29) (end 140.18 102.29) (width 0.3) (layer F.Cu) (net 34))
 (segment (start 143.26 103.35) (end 144.16 103.35) (width 0.3) (layer F.Cu) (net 35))
 (segment (start 140.76 104.29) (end 141.7 103.35) (width 0.3) (layer F.Cu) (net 35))
 (segment (start 137.74 104.29) (end 140.76 104.29) (width 0.3) (layer F.Cu) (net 35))
 (segment (start 141.7 103.35) (end 143.26 103.35) (width 0.3) (layer F.Cu) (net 35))
 (segment (start 142.86 104.15) (end 144.16 104.15) (width 0.3) (layer F.Cu) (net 36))
 (segment (start 137.74 106.29) (end 140.72 106.29) (width 0.3) (layer F.Cu) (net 36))
 (segment (start 140.72 106.29) (end 142.86 104.15) (width 0.3) (layer F.Cu) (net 36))
 (via (at 139.88 110.29) (size 1) (drill 0.4) (layers F.Cu B.Cu) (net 37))
 (segment (start 137.74 110.29) (end 139.88 110.29) (width 0.3) (layer F.Cu) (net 37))
 (segment (start 139.88 110.29) (end 139.88 106.84) (width 0.3) (layer B.Cu) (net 37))
 (via (at 146.09 104.81) (size 1) (drill 0.4) (layers F.Cu B.Cu) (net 37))
 (segment (start 139.88 106.84) (end 141.91 104.81) (width 0.3) (layer B.Cu) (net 37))
 (segment (start 141.91 104.81) (end 146.09 104.81) (width 0.3) (layer B.Cu) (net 37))
 (segment (start 145.95 104.95) (end 146.09 104.81) (width 0.3) (layer F.Cu) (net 37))
 (segment (start 144.16 104.95) (end 145.95 104.95) (width 0.3) (layer F.Cu) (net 37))
 (segment (start 139.99 108.29) (end 142.53 105.75) (width 0.3) (layer F.Cu) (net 38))
 (segment (start 137.74 108.29) (end 139.99 108.29) (width 0.3) (layer F.Cu) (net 38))
 (segment (start 142.53 105.75) (end 144.16 105.75) (width 0.3) (layer F.Cu) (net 38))
 (segment (start 143.26 106.55) (end 141.34 108.47) (width 0.3) (layer F.Cu) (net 39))
 (segment (start 144.16 106.55) (end 143.26 106.55) (width 0.3) (layer F.Cu) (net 39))
 (segment (start 141.34 108.47) (end 141.34 111.63) (width 0.3) (layer F.Cu) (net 39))
 (segment (start 140.68 112.29) (end 137.74 112.29) (width 0.3) (layer F.Cu) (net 39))
 (segment (start 141.34 111.63) (end 140.68 112.29) (width 0.3) (layer F.Cu) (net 39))
 (via (at 132.61 112.26) (size 1) (drill 0.4) (layers F.Cu B.Cu) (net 40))
 (segment (start 122.94 112.29) (end 132.58 112.29) (width 0.3) (layer F.Cu) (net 40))
 (segment (start 132.58 112.29) (end 132.61 112.26) (width 0.3) (layer F.Cu) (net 40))
 (segment (start 133.317106 112.26) (end 133.377106 112.32) (width 0.3) (layer B.Cu) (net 40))
 (segment (start 132.61 112.26) (end 133.317106 112.26) (width 0.3) (layer B.Cu) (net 40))
 (segment (start 133.377106 112.32) (end 140.72 112.32) (width 0.3) (layer B.Cu) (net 40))
 (segment (start 140.72 112.32) (end 141.72 111.32) (width 0.3) (layer B.Cu) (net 40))
 (segment (start 141.72 111.32) (end 141.72 108.04) (width 0.3) (layer B.Cu) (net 40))
 (via (at 146.22 107.32) (size 1) (drill 0.4) (layers F.Cu B.Cu) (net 40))
 (segment (start 141.72 108.04) (end 142.44 107.32) (width 0.3) (layer B.Cu) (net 40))
 (segment (start 142.44 107.32) (end 146.22 107.32) (width 0.3) (layer B.Cu) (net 40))
 (segment (start 144.19 107.32) (end 144.16 107.35) (width 0.3) (layer F.Cu) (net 40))
 (segment (start 146.22 107.32) (end 144.19 107.32) (width 0.3) (layer F.Cu) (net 40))
 (segment (start 122.94 114.29) (end 132.47 114.29) (width 0.3) (layer F.Cu) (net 41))
 (segment (start 132.47 114.29) (end 133.55 115.37) (width 0.3) (layer F.Cu) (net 41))
 (segment (start 133.55 115.37) (end 133.55 117.54) (width 0.3) (layer F.Cu) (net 41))
 (segment (start 133.55 117.54) (end 134.5 118.49) (width 0.3) (layer F.Cu) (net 41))
 (segment (start 134.5 118.49) (end 141.77 118.49) (width 0.3) (layer F.Cu) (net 41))
 (segment (start 141.77 118.49) (end 143.61 116.65) (width 0.3) (layer F.Cu) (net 41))
 (segment (start 143.61 116.65) (end 143.61 110.88) (width 0.3) (layer F.Cu) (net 41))
 (segment (start 144.09 110.4) (end 145.61 110.4) (width 0.3) (layer F.Cu) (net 41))
 (segment (start 143.61 110.88) (end 144.09 110.4) (width 0.3) (layer F.Cu) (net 41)))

